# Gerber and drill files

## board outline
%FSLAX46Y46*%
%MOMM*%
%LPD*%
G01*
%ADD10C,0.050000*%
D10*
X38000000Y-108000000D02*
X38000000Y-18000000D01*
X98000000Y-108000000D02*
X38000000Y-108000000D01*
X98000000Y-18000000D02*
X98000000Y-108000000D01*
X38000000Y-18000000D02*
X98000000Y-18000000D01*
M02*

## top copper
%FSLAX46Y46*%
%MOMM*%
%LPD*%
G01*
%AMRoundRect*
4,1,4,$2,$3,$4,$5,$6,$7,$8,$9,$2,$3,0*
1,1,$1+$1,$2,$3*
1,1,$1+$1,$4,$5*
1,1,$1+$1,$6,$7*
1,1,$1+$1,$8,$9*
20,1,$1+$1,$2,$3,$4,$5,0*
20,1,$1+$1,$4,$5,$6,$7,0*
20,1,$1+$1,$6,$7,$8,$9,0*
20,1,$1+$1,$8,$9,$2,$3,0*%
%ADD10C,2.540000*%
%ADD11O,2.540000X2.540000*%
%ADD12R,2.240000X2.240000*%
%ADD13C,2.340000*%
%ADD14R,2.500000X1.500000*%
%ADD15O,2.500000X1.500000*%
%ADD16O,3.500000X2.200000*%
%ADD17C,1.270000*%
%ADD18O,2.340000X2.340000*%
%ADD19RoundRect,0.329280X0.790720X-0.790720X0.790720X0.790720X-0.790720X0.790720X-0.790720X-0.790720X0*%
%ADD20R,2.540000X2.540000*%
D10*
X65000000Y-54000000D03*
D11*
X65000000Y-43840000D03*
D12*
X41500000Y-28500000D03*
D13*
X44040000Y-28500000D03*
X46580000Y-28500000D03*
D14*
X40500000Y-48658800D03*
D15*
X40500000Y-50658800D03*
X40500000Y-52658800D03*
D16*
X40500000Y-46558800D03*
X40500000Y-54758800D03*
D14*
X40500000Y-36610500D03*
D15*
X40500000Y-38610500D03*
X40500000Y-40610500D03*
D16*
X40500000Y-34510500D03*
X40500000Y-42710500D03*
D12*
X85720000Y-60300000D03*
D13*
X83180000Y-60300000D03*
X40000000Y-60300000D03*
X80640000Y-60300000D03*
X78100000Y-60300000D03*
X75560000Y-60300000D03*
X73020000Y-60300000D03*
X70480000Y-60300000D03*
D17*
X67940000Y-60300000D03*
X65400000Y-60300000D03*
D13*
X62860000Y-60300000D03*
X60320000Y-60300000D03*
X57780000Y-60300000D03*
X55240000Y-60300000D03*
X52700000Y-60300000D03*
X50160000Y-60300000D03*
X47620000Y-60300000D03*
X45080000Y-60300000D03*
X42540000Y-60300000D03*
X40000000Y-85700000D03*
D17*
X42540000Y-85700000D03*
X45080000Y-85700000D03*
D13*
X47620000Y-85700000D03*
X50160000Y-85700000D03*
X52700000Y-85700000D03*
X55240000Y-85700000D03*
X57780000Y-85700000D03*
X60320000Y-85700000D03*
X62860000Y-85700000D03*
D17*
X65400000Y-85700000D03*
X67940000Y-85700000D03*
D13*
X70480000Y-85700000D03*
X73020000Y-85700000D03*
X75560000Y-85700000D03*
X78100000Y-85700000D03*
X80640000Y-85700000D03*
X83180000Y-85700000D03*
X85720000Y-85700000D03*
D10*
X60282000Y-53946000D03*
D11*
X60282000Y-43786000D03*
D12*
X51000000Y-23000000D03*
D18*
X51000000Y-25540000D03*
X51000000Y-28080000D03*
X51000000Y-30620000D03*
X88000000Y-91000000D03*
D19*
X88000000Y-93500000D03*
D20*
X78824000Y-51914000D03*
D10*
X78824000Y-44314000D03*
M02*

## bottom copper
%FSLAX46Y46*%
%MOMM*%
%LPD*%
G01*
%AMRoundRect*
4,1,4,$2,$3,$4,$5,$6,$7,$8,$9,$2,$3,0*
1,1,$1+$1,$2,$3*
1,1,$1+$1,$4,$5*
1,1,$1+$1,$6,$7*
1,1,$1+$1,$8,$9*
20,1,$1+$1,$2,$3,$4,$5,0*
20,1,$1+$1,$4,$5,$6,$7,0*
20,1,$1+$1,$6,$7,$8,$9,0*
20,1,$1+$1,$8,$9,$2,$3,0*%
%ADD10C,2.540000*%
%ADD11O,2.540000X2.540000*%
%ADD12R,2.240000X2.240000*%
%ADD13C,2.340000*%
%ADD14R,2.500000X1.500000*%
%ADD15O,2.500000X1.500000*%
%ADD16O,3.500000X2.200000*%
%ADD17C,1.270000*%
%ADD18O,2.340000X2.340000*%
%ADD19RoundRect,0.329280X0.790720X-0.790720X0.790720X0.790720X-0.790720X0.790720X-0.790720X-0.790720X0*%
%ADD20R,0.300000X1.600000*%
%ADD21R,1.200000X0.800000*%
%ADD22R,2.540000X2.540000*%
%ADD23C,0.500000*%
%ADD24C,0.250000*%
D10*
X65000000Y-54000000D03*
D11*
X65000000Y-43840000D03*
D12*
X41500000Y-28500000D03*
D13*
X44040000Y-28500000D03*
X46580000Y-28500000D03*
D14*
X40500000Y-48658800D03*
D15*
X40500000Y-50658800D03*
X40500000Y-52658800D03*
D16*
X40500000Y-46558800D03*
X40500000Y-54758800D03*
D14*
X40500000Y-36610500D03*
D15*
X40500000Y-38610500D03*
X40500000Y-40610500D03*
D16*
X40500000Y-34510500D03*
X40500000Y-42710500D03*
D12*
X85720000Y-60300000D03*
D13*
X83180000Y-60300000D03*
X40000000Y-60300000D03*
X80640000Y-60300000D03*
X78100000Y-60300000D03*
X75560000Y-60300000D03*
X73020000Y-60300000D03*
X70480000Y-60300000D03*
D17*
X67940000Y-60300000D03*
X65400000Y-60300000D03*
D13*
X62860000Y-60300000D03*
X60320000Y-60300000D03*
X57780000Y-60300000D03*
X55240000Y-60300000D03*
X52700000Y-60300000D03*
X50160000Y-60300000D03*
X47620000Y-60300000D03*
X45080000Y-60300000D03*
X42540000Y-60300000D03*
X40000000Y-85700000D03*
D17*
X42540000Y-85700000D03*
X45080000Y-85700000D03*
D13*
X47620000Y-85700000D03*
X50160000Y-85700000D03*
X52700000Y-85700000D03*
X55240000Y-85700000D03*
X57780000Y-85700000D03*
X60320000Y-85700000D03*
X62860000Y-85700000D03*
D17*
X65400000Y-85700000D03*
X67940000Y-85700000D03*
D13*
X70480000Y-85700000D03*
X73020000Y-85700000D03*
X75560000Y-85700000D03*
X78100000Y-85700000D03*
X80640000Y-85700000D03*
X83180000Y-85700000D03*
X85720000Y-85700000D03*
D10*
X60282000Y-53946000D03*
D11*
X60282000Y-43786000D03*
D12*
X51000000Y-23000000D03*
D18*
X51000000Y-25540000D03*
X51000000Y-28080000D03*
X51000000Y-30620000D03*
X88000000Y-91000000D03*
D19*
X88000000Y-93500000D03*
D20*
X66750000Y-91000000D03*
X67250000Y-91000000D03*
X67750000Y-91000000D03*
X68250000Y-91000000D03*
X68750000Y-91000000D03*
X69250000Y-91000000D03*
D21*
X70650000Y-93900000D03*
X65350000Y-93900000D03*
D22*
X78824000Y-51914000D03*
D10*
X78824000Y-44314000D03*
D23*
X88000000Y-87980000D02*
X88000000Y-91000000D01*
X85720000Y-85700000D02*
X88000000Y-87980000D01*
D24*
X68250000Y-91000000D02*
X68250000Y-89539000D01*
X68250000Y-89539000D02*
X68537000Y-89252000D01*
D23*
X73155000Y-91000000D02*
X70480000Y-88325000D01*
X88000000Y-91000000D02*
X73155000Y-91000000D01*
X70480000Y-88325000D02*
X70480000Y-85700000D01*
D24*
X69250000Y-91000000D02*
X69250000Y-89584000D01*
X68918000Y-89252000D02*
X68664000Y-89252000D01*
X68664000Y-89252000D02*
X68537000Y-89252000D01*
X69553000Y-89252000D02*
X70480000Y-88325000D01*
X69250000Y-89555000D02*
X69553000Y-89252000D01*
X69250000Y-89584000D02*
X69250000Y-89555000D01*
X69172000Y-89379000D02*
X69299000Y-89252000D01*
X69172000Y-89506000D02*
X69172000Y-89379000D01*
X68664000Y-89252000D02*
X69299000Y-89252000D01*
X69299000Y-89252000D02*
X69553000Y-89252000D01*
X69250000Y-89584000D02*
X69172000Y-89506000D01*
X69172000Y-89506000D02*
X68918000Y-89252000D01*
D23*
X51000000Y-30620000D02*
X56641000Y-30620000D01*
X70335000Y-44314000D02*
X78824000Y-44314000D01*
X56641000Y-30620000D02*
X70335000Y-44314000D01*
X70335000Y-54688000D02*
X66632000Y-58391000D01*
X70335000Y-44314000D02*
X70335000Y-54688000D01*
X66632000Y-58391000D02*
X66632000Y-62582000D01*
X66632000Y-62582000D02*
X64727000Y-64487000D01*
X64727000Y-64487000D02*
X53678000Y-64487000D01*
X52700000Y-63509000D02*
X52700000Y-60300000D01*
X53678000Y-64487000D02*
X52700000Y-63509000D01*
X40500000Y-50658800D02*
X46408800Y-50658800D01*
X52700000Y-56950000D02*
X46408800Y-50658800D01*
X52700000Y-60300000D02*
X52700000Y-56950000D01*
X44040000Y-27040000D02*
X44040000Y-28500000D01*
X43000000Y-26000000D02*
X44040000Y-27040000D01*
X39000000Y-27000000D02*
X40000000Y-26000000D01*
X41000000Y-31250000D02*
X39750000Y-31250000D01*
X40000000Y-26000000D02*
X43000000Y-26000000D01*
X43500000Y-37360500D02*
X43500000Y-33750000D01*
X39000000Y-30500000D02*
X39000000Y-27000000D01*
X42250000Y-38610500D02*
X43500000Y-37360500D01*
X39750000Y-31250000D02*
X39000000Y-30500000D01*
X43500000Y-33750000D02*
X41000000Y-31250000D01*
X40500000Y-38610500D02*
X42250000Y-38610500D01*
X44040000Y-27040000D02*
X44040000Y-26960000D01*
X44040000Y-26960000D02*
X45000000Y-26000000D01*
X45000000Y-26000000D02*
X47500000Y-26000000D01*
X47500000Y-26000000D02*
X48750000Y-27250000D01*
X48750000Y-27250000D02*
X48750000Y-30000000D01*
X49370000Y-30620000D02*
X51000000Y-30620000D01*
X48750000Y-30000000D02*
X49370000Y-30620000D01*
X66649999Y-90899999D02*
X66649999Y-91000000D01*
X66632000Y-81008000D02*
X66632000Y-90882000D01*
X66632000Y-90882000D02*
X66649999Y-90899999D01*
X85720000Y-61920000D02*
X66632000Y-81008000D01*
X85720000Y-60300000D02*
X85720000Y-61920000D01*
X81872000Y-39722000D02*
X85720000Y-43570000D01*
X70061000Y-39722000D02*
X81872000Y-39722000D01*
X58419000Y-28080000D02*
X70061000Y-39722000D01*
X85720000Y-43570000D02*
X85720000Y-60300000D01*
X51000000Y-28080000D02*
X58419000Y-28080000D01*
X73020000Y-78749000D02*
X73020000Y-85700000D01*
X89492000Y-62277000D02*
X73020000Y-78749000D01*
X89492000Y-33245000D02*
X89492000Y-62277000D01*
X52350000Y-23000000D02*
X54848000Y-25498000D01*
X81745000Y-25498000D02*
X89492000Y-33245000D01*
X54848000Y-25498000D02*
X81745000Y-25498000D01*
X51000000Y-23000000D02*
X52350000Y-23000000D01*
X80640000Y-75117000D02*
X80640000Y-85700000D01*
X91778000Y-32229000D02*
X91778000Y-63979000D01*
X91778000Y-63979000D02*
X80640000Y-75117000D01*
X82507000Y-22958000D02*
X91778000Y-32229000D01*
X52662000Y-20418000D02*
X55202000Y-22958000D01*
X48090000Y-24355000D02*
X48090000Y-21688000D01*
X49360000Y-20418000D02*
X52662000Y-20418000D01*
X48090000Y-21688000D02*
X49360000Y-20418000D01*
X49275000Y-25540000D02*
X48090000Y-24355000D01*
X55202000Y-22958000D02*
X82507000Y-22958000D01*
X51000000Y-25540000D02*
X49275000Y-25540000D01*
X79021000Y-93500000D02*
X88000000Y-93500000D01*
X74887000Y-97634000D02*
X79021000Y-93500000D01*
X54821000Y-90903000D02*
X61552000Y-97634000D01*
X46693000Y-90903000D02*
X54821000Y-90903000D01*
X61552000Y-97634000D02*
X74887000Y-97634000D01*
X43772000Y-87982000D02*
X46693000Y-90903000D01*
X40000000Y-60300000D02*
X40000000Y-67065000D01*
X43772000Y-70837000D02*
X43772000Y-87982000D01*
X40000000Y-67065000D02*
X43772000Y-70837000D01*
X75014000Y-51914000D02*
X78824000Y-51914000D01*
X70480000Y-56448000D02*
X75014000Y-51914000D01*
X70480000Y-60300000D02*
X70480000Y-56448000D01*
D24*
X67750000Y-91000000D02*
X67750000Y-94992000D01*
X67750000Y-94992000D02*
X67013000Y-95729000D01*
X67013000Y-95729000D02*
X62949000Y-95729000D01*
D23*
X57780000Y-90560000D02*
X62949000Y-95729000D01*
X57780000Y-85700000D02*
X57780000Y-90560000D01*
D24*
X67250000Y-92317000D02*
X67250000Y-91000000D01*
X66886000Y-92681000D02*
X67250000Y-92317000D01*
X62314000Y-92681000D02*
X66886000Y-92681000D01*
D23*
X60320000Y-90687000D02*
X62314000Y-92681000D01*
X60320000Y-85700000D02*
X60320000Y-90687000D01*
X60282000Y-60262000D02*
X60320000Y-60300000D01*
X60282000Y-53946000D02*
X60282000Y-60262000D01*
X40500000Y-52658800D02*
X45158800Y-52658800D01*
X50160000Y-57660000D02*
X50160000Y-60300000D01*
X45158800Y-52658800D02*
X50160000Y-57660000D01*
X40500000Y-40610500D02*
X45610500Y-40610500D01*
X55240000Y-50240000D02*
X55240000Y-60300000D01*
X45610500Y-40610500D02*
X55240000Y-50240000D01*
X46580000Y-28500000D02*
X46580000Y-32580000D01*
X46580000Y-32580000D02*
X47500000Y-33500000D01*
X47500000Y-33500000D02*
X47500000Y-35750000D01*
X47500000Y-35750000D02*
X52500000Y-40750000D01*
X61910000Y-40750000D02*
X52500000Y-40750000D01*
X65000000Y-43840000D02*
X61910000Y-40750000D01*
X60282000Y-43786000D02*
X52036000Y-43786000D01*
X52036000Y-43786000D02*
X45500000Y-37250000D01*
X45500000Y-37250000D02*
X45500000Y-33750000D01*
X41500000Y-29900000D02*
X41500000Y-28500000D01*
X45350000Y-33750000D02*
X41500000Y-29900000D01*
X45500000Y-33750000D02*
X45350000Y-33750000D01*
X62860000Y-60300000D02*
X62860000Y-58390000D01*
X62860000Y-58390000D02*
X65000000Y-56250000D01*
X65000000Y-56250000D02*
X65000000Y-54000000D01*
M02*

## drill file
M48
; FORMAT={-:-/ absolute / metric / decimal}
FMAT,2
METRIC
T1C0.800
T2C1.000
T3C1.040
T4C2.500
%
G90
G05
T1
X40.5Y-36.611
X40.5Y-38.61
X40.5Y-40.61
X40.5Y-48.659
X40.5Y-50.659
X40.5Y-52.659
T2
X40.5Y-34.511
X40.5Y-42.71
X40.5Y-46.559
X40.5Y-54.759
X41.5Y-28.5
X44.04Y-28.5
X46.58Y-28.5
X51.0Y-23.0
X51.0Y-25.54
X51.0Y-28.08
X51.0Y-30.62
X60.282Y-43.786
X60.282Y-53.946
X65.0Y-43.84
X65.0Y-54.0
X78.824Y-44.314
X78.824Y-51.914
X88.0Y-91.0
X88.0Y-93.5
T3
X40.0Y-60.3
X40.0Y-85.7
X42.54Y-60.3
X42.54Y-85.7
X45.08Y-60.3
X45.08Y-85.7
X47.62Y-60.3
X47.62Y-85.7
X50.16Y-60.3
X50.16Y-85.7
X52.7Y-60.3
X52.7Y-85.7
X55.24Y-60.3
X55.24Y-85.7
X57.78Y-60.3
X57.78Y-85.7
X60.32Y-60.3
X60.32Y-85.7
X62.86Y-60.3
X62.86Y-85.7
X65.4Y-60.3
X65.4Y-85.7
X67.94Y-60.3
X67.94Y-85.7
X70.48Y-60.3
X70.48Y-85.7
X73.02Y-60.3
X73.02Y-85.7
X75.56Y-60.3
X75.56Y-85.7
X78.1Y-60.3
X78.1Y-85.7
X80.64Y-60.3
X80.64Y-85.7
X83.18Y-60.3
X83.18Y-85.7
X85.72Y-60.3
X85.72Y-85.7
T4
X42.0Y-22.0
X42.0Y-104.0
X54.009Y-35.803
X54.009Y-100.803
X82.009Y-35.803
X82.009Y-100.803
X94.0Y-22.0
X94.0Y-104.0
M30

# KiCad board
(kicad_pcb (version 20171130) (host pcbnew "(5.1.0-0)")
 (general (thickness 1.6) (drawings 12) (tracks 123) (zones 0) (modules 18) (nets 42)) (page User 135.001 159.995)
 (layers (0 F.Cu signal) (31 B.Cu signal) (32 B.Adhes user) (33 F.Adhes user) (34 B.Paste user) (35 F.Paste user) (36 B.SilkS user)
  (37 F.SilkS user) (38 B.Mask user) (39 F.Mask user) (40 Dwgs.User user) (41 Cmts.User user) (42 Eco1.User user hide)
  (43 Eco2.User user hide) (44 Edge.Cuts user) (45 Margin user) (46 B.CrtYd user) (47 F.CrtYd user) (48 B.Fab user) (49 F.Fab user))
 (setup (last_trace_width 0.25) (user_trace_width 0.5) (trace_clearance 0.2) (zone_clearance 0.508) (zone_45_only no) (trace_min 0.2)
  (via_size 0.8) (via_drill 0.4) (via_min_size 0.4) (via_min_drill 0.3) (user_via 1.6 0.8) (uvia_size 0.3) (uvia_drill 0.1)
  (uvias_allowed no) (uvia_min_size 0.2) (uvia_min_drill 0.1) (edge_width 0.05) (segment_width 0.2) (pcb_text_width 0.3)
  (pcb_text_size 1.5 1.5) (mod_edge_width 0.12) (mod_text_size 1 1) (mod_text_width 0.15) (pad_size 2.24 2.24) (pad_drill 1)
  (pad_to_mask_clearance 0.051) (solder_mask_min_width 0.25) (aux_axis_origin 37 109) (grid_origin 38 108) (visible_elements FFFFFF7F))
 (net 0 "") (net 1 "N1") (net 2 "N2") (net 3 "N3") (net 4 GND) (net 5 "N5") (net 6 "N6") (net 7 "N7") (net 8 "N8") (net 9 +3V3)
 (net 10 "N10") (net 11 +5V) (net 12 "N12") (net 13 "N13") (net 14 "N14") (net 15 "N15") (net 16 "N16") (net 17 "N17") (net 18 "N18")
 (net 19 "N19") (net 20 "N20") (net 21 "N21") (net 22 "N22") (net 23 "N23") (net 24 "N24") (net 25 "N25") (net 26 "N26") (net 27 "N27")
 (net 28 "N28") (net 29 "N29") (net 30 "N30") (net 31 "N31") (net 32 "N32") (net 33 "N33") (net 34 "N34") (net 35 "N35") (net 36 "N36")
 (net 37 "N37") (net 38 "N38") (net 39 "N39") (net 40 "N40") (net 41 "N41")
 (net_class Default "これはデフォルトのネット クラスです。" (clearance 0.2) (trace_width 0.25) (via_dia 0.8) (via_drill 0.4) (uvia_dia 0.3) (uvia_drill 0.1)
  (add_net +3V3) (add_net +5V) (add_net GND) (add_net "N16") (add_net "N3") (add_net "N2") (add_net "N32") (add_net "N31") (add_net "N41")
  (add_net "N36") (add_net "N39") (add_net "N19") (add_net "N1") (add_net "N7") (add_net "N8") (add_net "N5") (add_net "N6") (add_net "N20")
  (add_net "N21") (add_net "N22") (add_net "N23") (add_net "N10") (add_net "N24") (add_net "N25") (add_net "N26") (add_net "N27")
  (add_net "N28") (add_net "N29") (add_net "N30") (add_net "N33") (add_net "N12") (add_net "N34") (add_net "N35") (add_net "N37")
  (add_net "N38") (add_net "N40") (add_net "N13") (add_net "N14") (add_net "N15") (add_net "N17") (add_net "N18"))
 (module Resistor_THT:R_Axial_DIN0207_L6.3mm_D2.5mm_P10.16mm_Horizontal (layer F.Cu) (at 65 54 90)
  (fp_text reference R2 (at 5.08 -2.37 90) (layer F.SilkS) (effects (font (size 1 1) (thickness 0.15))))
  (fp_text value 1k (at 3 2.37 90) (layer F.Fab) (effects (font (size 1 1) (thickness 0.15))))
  (pad 1 thru_hole circle (at 0 0 90) (size 2.54 2.54) (drill 1) (layers *.Cu *.Mask) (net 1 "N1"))
  (pad 2 thru_hole oval (at 10.16 0 90) (size 2.54 2.54) (drill 1) (layers *.Cu *.Mask) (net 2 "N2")))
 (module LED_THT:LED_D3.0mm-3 (layer F.Cu) (at 41.5 28.5)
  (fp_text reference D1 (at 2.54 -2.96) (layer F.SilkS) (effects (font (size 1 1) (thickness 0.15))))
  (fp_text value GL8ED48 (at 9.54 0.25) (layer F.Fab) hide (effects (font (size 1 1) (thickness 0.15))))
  (pad 1 thru_hole rect (at 0 0) (size 2.24 2.24) (drill 1) (layers *.Cu *.Mask) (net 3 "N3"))
  (pad 2 thru_hole circle (at 2.54 0) (size 2.34 2.34) (drill 1) (layers *.Cu *.Mask) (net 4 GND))
  (pad 3 thru_hole circle (at 5.08 0) (size 2.34 2.34) (drill 1) (layers *.Cu *.Mask) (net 2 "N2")))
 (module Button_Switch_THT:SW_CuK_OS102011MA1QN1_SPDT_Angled (layer F.Cu) (at 40.5 48.6588 270)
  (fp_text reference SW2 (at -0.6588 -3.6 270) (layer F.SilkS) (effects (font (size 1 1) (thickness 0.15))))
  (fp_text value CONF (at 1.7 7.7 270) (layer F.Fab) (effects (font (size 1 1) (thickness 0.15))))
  (pad 1 thru_hole rect (at 0 0 270) (size 1.5 2.5) (drill 0.8) (layers *.Cu *.Mask) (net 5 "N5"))
  (pad 2 thru_hole oval (at 2 0 270) (size 1.5 2.5) (drill 0.8) (layers *.Cu *.Mask) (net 4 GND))
  (pad 3 thru_hole oval (at 4 0 270) (size 1.5 2.5) (drill 0.8) (layers *.Cu *.Mask) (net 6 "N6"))
  (pad "" thru_hole oval (at -2.1 0 270) (size 2.2 3.5) (drill 1) (layers *.Cu *.Mask))
  (pad "" thru_hole oval (at 6.1 0 270) (size 2.2 3.5) (drill 1) (layers *.Cu *.Mask)))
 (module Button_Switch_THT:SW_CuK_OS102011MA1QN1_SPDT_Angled (layer F.Cu) (at 40.5 36.6105 270)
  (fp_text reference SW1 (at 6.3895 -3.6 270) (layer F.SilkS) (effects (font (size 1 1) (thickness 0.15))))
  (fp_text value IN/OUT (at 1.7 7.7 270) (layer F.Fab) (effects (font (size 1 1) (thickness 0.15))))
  (pad 1 thru_hole rect (at 0 0 270) (size 1.5 2.5) (drill 0.8) (layers *.Cu *.Mask) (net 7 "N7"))
  (pad 2 thru_hole oval (at 2 0 270) (size 1.5 2.5) (drill 0.8) (layers *.Cu *.Mask) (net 4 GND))
  (pad 3 thru_hole oval (at 4 0 270) (size 1.5 2.5) (drill 0.8) (layers *.Cu *.Mask) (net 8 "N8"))
  (pad "" thru_hole oval (at -2.1 0 270) (size 2.2 3.5) (drill 1) (layers *.Cu *.Mask))
  (pad "" thru_hole oval (at 6.1 0 270) (size 2.2 3.5) (drill 1) (layers *.Cu *.Mask)))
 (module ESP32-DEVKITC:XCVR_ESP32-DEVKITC (layer F.Cu) (at 66.26 73 270)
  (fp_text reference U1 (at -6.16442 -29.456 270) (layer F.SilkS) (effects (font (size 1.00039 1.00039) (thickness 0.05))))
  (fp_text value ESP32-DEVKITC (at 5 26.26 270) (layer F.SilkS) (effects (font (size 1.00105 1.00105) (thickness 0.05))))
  (pad 1 thru_hole rect (at -12.7 -19.46 270) (size 2.24 2.24) (drill 1.04) (layers *.Cu *.Mask) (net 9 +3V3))
  (pad 2 thru_hole circle (at -12.7 -16.92 270) (size 2.34 2.34) (drill 1.04) (layers *.Cu *.Mask) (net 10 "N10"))
  (pad 19 thru_hole circle (at -12.7 26.26 270) (size 2.34 2.34) (drill 1.04) (layers *.Cu *.Mask) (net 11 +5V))
  (pad 3 thru_hole circle (at -12.7 -14.38 270) (size 2.34 2.34) (drill 1.04) (layers *.Cu *.Mask) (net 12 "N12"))
  (pad 4 thru_hole circle (at -12.7 -11.84 270) (size 2.34 2.34) (drill 1.04) (layers *.Cu *.Mask) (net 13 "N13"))
  (pad 5 thru_hole circle (at -12.7 -9.3 270) (size 2.34 2.34) (drill 1.04) (layers *.Cu *.Mask) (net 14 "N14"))
  (pad 6 thru_hole circle (at -12.7 -6.76 270) (size 2.34 2.34) (drill 1.04) (layers *.Cu *.Mask) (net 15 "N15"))
  (pad 7 thru_hole circle (at -12.7 -4.22 270) (size 2.34 2.34) (drill 1.04) (layers *.Cu *.Mask) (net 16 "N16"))
  (pad 8 thru_hole circle (at -12.7 -1.68 270) (size 1.27 1.27) (drill 1.04) (layers *.Cu *.Mask) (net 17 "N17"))
  (pad 9 thru_hole circle (at -12.7 0.86 270) (size 1.27 1.27) (drill 1.04) (layers *.Cu *.Mask) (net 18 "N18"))
  (pad 10 thru_hole circle (at -12.7 3.4 270) (size 2.34 2.34) (drill 1.04) (layers *.Cu *.Mask) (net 1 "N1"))
  (pad 11 thru_hole circle (at -12.7 5.94 270) (size 2.34 2.34) (drill 1.04) (layers *.Cu *.Mask) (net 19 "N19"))
  (pad 12 thru_hole circle (at -12.7 8.48 270) (size 2.34 2.34) (drill 1.04) (layers *.Cu *.Mask) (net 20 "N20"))
  (pad 13 thru_hole circle (at -12.7 11.02 270) (size 2.34 2.34) (drill 1.04) (layers *.Cu *.Mask) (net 8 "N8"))
  (pad 14 thru_hole circle (at -12.7 13.56 270) (size 2.34 2.34) (drill 1.04) (layers *.Cu *.Mask) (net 4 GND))
  (pad 15 thru_hole circle (at -12.7 16.1 270) (size 2.34 2.34) (drill 1.04) (layers *.Cu *.Mask) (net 6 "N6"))
  (pad 16 thru_hole circle (at -12.7 18.64 270) (size 2.34 2.34) (drill 1.04) (layers *.Cu *.Mask) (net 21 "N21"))
  (pad 17 thru_hole circle (at -12.7 21.18 270) (size 2.34 2.34) (drill 1.04) (layers *.Cu *.Mask) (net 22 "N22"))
  (pad 18 thru_hole circle (at -12.7 23.72 270) (size 2.34 2.34) (drill 1.04) (layers *.Cu *.Mask) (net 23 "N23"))
  (pad 20 thru_hole circle (at 12.7 26.26 90) (size 2.34 2.34) (drill 1.04) (layers *.Cu *.Mask) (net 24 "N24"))
  (pad 21 thru_hole circle (at 12.7 23.72 90) (size 1.27 1.27) (drill 1.04) (layers *.Cu *.Mask) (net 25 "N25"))
  (pad 22 thru_hole circle (at 12.7 21.18 90) (size 1.27 1.27) (drill 1.04) (layers *.Cu *.Mask) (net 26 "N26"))
  (pad 23 thru_hole circle (at 12.7 18.64 90) (size 2.34 2.34) (drill 1.04) (layers *.Cu *.Mask) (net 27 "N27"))
  (pad 24 thru_hole circle (at 12.7 16.1 90) (size 2.34 2.34) (drill 1.04) (layers *.Cu *.Mask) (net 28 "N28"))
  (pad 25 thru_hole circle (at 12.7 13.56 90) (size 2.34 2.34) (drill 1.04) (layers *.Cu *.Mask) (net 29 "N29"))
  (pad 26 thru_hole circle (at 12.7 11.02 90) (size 2.34 2.34) (drill 1.04) (layers *.Cu *.Mask) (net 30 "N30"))
  (pad 27 thru_hole circle (at 12.7 8.48 90) (size 2.34 2.34) (drill 1.04) (layers *.Cu *.Mask) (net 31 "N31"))
  (pad 28 thru_hole circle (at 12.7 5.94 90) (size 2.34 2.34) (drill 1.04) (layers *.Cu *.Mask) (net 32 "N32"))
  (pad 29 thru_hole circle (at 12.7 3.4 90) (size 2.34 2.34) (drill 1.04) (layers *.Cu *.Mask) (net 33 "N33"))
  (pad 30 thru_hole circle (at 12.7 0.86 90) (size 1.27 1.27) (drill 1.04) (layers *.Cu *.Mask) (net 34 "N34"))
  (pad 31 thru_hole circle (at 12.7 -1.68 90) (size 1.27 1.27) (drill 1.04) (layers *.Cu *.Mask) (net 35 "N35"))
  (pad 32 thru_hole circle (at 12.7 -4.22 90) (size 2.34 2.34) (drill 1.04) (layers *.Cu *.Mask) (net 4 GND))
  (pad 33 thru_hole circle (at 12.7 -6.76 90) (size 2.34 2.34) (drill 1.04) (layers *.Cu *.Mask) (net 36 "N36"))
  (pad 34 thru_hole circle (at 12.7 -9.3 90) (size 2.34 2.34) (drill 1.04) (layers *.Cu *.Mask) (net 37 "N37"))
  (pad 35 thru_hole circle (at 12.7 -11.84 90) (size 2.34 2.34) (drill 1.04) (layers *.Cu *.Mask) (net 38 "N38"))
  (pad 36 thru_hole circle (at 12.7 -14.38 90) (size 2.34 2.34) (drill 1.04) (layers *.Cu *.Mask) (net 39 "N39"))
  (pad 37 thru_hole circle (at 12.7 -16.92 90) (size 2.34 2.34) (drill 1.04) (layers *.Cu *.Mask) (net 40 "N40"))
  (pad 38 thru_hole circle (at 12.7 -19.46 90) (size 2.34 2.34) (drill 1.04) (layers *.Cu *.Mask) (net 4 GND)))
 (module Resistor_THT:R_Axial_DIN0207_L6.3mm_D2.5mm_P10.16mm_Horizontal (layer F.Cu) (at 60.282 53.946 90)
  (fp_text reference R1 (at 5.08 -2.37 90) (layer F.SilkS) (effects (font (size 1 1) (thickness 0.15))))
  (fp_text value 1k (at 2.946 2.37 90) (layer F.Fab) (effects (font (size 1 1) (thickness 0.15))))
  (pad 1 thru_hole circle (at 0 0 90) (size 2.54 2.54) (drill 1) (layers *.Cu *.Mask) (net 19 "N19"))
  (pad 2 thru_hole oval (at 10.16 0 90) (size 2.54 2.54) (drill 1) (layers *.Cu *.Mask) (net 3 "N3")))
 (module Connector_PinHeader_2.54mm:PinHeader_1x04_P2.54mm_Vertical (layer F.Cu) (at 51 23)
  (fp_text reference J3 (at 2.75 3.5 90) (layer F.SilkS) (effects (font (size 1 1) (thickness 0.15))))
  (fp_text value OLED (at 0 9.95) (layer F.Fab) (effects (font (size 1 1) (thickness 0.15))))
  (pad 1 thru_hole rect (at 0 0) (size 2.24 2.24) (drill 1) (layers *.Cu *.Mask) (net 36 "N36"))
  (pad 2 thru_hole oval (at 0 2.54) (size 2.34 2.34) (drill 1) (layers *.Cu *.Mask) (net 39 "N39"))
  (pad 3 thru_hole oval (at 0 5.08) (size 2.34 2.34) (drill 1) (layers *.Cu *.Mask) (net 9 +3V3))
  (pad 4 thru_hole oval (at 0 7.62) (size 2.34 2.34) (drill 1) (layers *.Cu *.Mask) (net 4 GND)))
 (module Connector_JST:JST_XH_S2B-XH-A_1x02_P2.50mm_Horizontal (layer F.Cu) (at 88 93.5 90)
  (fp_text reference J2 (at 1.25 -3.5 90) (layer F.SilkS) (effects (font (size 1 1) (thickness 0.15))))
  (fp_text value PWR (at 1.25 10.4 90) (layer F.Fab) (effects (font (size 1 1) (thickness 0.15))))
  (pad 2 thru_hole oval (at 2.5 0 90) (size 2.34 2.34) (drill 1) (layers *.Cu *.Mask) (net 4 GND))
  (pad 1 thru_hole roundrect (at 0 0 90) (size 2.24 2.24) (drill 1) (layers *.Cu *.Mask) (roundrect_rratio 0.147) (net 11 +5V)))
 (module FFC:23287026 (layer B.Cu) (at 68 92.8 180)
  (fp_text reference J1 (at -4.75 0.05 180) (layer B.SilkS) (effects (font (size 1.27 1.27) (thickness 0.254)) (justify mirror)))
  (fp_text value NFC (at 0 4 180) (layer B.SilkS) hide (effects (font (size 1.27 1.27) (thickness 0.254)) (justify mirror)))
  (pad 1 smd rect (at 1.25 1.8 180) (size 0.3 1.6) (layers B.Cu B.Paste B.Mask) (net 9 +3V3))
  (pad 2 smd rect (at 0.75 1.8 180) (size 0.3 1.6) (layers B.Cu B.Paste B.Mask) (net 32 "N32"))
  (pad 3 smd rect (at 0.25 1.8 180) (size 0.3 1.6) (layers B.Cu B.Paste B.Mask) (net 31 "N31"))
  (pad 4 smd rect (at -0.25 1.8 180) (size 0.3 1.6) (layers B.Cu B.Paste B.Mask) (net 4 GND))
  (pad 5 smd rect (at -0.75 1.8 180) (size 0.3 1.6) (layers B.Cu B.Paste B.Mask) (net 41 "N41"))
  (pad 6 smd rect (at -1.25 1.8 180) (size 0.3 1.6) (layers B.Cu B.Paste B.Mask) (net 4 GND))
  (pad MP1 smd rect (at -2.65 -1.1 180) (size 1.2 0.8) (layers B.Cu B.Paste B.Mask))
  (pad MP2 smd rect (at 2.65 -1.1 180) (size 1.2 0.8) (layers B.Cu B.Paste B.Mask)))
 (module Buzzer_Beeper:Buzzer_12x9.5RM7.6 (layer F.Cu) (at 78.824 51.914 90)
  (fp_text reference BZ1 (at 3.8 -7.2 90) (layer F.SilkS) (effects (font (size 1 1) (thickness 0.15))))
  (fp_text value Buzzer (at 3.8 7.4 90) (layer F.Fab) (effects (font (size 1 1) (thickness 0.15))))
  (pad 1 thru_hole rect (at 0 0 90) (size 2.54 2.54) (drill 1) (layers *.Cu *.Mask) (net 16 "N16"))
  (pad 2 thru_hole circle (at 7.6 0 90) (size 2.54 2.54) (drill 1) (layers *.Cu *.Mask) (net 4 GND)))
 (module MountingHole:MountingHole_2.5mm (layer F.Cu) (at 42 104)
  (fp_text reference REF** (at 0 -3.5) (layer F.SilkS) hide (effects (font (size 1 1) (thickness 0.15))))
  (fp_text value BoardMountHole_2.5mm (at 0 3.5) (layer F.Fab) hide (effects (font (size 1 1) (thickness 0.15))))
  (pad 1 np_thru_hole circle (at 0 0) (size 2.5 2.5) (drill 2.5) (layers *.Cu *.Mask)))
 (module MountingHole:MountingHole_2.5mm (layer F.Cu) (at 94 104)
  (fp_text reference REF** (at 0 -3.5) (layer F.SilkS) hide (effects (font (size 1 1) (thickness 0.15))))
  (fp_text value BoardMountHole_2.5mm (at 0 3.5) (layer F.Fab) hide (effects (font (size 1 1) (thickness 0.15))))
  (pad 1 np_thru_hole circle (at 0 0) (size 2.5 2.5) (drill 2.5) (layers *.Cu *.Mask)))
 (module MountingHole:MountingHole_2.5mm (layer F.Cu) (at 94 22)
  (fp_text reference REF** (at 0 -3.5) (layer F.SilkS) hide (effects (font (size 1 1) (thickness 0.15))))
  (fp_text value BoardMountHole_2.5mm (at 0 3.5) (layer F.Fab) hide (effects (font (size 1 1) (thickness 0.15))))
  (pad 1 np_thru_hole circle (at 0 0) (size 2.5 2.5) (drill 2.5) (layers *.Cu *.Mask)))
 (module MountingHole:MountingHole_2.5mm (layer F.Cu) (at 42 22)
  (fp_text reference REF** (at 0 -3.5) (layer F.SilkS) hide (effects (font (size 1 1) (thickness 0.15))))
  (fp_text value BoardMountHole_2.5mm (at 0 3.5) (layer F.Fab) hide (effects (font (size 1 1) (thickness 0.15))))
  (pad 1 np_thru_hole circle (at 0 0) (size 2.5 2.5) (drill 2.5) (layers *.Cu *.Mask)))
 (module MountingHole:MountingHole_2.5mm (layer F.Cu) (at 54.008576 35.802609 90)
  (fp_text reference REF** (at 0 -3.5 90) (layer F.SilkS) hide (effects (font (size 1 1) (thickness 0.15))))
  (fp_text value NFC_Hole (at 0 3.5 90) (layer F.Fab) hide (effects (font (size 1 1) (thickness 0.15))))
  (pad 1 np_thru_hole circle (at 0 0 90) (size 2.5 2.5) (drill 2.5) (layers *.Cu *.Mask)))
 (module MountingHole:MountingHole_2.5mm (layer F.Cu) (at 82.008576 100.802609 90)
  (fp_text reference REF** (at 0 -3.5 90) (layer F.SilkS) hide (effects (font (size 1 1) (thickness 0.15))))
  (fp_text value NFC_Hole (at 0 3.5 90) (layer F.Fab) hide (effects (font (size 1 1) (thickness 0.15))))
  (pad 1 np_thru_hole circle (at 0 0 90) (size 2.5 2.5) (drill 2.5) (layers *.Cu *.Mask)))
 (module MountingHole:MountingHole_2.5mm (layer F.Cu) (at 82.008576 35.802609 90)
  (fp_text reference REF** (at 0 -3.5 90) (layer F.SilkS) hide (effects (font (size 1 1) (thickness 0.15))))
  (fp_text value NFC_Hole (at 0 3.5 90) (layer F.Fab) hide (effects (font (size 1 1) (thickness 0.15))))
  (pad 1 np_thru_hole circle (at 0 0 90) (size 2.5 2.5) (drill 2.5) (layers *.Cu *.Mask)))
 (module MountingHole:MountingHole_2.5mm (layer F.Cu) (at 54.008576 100.802609 90)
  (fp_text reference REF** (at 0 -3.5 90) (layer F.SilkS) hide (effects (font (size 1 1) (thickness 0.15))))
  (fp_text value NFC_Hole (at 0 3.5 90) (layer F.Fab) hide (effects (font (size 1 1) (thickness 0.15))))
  (pad 1 np_thru_hole circle (at 0 0 90) (size 2.5 2.5) (drill 2.5) (layers *.Cu *.Mask)))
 (gr_line (start 38 108) (end 38 18) (layer Edge.Cuts) (width 0.05))
 (gr_line (start 98 108) (end 38 108) (layer Edge.Cuts) (width 0.05))
 (gr_line (start 98 18) (end 98 108) (layer Edge.Cuts) (width 0.05))
 (gr_line (start 38 18) (end 98 18) (layer Edge.Cuts) (width 0.05))
 (segment (start 88 87.98) (end 88 91) (width 0.5) (layer B.Cu) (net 4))
 (segment (start 85.72 85.7) (end 88 87.98) (width 0.5) (layer B.Cu) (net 4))
 (segment (start 68.25 91) (end 68.25 89.539) (width 0.25) (layer B.Cu) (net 4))
 (segment (start 68.25 89.539) (end 68.537 89.252) (width 0.25) (layer B.Cu) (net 4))
 (segment (start 73.155 91) (end 70.48 88.325) (width 0.5) (layer B.Cu) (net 4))
 (segment (start 88 91) (end 73.155 91) (width 0.5) (layer B.Cu) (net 4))
 (segment (start 70.48 88.325) (end 70.48 85.7) (width 0.5) (layer B.Cu) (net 4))
 (segment (start 69.25 91) (end 69.25 89.584) (width 0.25) (layer B.Cu) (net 4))
 (segment (start 68.918 89.252) (end 68.664 89.252) (width 0.25) (layer B.Cu) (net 4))
 (segment (start 68.664 89.252) (end 68.537 89.252) (width 0.25) (layer B.Cu) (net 4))
 (segment (start 69.553 89.252) (end 70.48 88.325) (width 0.25) (layer B.Cu) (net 4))
 (segment (start 69.25 89.555) (end 69.553 89.252) (width 0.25) (layer B.Cu) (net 4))
 (segment (start 69.25 89.584) (end 69.25 89.555) (width 0.25) (layer B.Cu) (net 4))
 (segment (start 69.172 89.379) (end 69.299 89.252) (width 0.25) (layer B.Cu) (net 4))
 (segment (start 69.172 89.506) (end 69.172 89.379) (width 0.25) (layer B.Cu) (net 4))
 (segment (start 68.664 89.252) (end 69.299 89.252) (width 0.25) (layer B.Cu) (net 4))
 (segment (start 69.299 89.252) (end 69.553 89.252) (width 0.25) (layer B.Cu) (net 4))
 (segment (start 69.25 89.584) (end 69.172 89.506) (width 0.25) (layer B.Cu) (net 4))
 (segment (start 69.172 89.506) (end 68.918 89.252) (width 0.25) (layer B.Cu) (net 4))
 (segment (start 51 30.62) (end 56.641 30.62) (width 0.5) (layer B.Cu) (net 4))
 (segment (start 70.335 44.314) (end 78.824 44.314) (width 0.5) (layer B.Cu) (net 4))
 (segment (start 56.641 30.62) (end 70.335 44.314) (width 0.5) (layer B.Cu) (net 4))
 (segment (start 70.335 54.688) (end 66.632 58.391) (width 0.5) (layer B.Cu) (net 4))
 (segment (start 70.335 44.314) (end 70.335 54.688) (width 0.5) (layer B.Cu) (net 4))
 (segment (start 66.632 58.391) (end 66.632 62.582) (width 0.5) (layer B.Cu) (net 4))
 (segment (start 66.632 62.582) (end 64.727 64.487) (width 0.5) (layer B.Cu) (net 4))
 (segment (start 64.727 64.487) (end 53.678 64.487) (width 0.5) (layer B.Cu) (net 4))
 (segment (start 52.7 63.509) (end 52.7 60.3) (width 0.5) (layer B.Cu) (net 4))
 (segment (start 53.678 64.487) (end 52.7 63.509) (width 0.5) (layer B.Cu) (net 4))
 (segment (start 40.5 50.6588) (end 46.4088 50.6588) (width 0.5) (layer B.Cu) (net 4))
 (segment (start 52.7 56.95) (end 46.4088 50.6588) (width 0.5) (layer B.Cu) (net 4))
 (segment (start 52.7 60.3) (end 52.7 56.95) (width 0.5) (layer B.Cu) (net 4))
 (segment (start 44.04 27.04) (end 44.04 28.5) (width 0.5) (layer B.Cu) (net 4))
 (segment (start 43 26) (end 44.04 27.04) (width 0.5) (layer B.Cu) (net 4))
 (segment (start 39 27) (end 40 26) (width 0.5) (layer B.Cu) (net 4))
 (segment (start 41 31.25) (end 39.75 31.25) (width 0.5) (layer B.Cu) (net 4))
 (segment (start 40 26) (end 43 26) (width 0.5) (layer B.Cu) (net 4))
 (segment (start 43.5 37.3605) (end 43.5 33.75) (width 0.5) (layer B.Cu) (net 4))
 (segment (start 39 30.5) (end 39 27) (width 0.5) (layer B.Cu) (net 4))
 (segment (start 42.25 38.6105) (end 43.5 37.3605) (width 0.5) (layer B.Cu) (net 4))
 (segment (start 39.75 31.25) (end 39 30.5) (width 0.5) (layer B.Cu) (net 4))
 (segment (start 43.5 33.75) (end 41 31.25) (width 0.5) (layer B.Cu) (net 4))
 (segment (start 40.5 38.6105) (end 42.25 38.6105) (width 0.5) (layer B.Cu) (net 4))
 (segment (start 44.04 27.04) (end 44.04 26.96) (width 0.5) (layer B.Cu) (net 4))
 (segment (start 44.04 26.96) (end 45 26) (width 0.5) (layer B.Cu) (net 4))
 (segment (start 45 26) (end 47.5 26) (width 0.5) (layer B.Cu) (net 4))
 (segment (start 47.5 26) (end 48.75 27.25) (width 0.5) (layer B.Cu) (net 4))
 (segment (start 48.75 27.25) (end 48.75 30) (width 0.5) (layer B.Cu) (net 4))
 (segment (start 49.37 30.62) (end 51 30.62) (width 0.5) (layer B.Cu) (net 4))
 (segment (start 48.75 30) (end 49.37 30.62) (width 0.5) (layer B.Cu) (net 4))
 (segment (start 66.649999 90.899999) (end 66.649999 91) (width 0.5) (layer B.Cu) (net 9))
 (segment (start 66.632 81.008) (end 66.632 90.882) (width 0.5) (layer B.Cu) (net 9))
 (segment (start 66.632 90.882) (end 66.649999 90.899999) (width 0.5) (layer B.Cu) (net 9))
 (segment (start 85.72 61.92) (end 66.632 81.008) (width 0.5) (layer B.Cu) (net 9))
 (segment (start 85.72 60.3) (end 85.72 61.92) (width 0.5) (layer B.Cu) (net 9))
 (segment (start 81.872 39.722) (end 85.72 43.57) (width 0.5) (layer B.Cu) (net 9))
 (segment (start 70.061 39.722) (end 81.872 39.722) (width 0.5) (layer B.Cu) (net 9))
 (segment (start 58.419 28.08) (end 70.061 39.722) (width 0.5) (layer B.Cu) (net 9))
 (segment (start 85.72 43.57) (end 85.72 60.3) (width 0.5) (layer B.Cu) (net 9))
 (segment (start 51 28.08) (end 58.419 28.08) (width 0.5) (layer B.Cu) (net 9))
 (segment (start 73.02 78.749) (end 73.02 85.7) (width 0.5) (layer B.Cu) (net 36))
 (segment (start 89.492 62.277) (end 73.02 78.749) (width 0.5) (layer B.Cu) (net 36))
 (segment (start 89.492 33.245) (end 89.492 62.277) (width 0.5) (layer B.Cu) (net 36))
 (segment (start 52.35 23) (end 54.848 25.498) (width 0.5) (layer B.Cu) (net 36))
 (segment (start 81.745 25.498) (end 89.492 33.245) (width 0.5) (layer B.Cu) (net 36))
 (segment (start 54.848 25.498) (end 81.745 25.498) (width 0.5) (layer B.Cu) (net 36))
 (segment (start 51 23) (end 52.35 23) (width 0.5) (layer B.Cu) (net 36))
 (segment (start 80.64 75.117) (end 80.64 85.7) (width 0.5) (layer B.Cu) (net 39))
 (segment (start 91.778 32.229) (end 91.778 63.979) (width 0.5) (layer B.Cu) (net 39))
 (segment (start 91.778 63.979) (end 80.64 75.117) (width 0.5) (layer B.Cu) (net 39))
 (segment (start 82.507 22.958) (end 91.778 32.229) (width 0.5) (layer B.Cu) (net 39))
 (segment (start 52.662 20.418) (end 55.202 22.958) (width 0.5) (layer B.Cu) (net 39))
 (segment (start 48.09 24.355) (end 48.09 21.688) (width 0.5) (layer B.Cu) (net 39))
 (segment (start 49.36 20.418) (end 52.662 20.418) (width 0.5) (layer B.Cu) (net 39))
 (segment (start 48.09 21.688) (end 49.36 20.418) (width 0.5) (layer B.Cu) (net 39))
 (segment (start 49.275 25.54) (end 48.09 24.355) (width 0.5) (layer B.Cu) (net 39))
 (segment (start 55.202 22.958) (end 82.507 22.958) (width 0.5) (layer B.Cu) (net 39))
 (segment (start 51 25.54) (end 49.275 25.54) (width 0.5) (layer B.Cu) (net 39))
 (segment (start 79.021 93.5) (end 88 93.5) (width 0.5) (layer B.Cu) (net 11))
 (segment (start 74.887 97.634) (end 79.021 93.5) (width 0.5) (layer B.Cu) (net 11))
 (segment (start 54.821 90.903) (end 61.552 97.634) (width 0.5) (layer B.Cu) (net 11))
 (segment (start 46.693 90.903) (end 54.821 90.903) (width 0.5) (layer B.Cu) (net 11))
 (segment (start 61.552 97.634) (end 74.887 97.634) (width 0.5) (layer B.Cu) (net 11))
 (segment (start 43.772 87.982) (end 46.693 90.903) (width 0.5) (layer B.Cu) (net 11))
 (segment (start 40 60.3) (end 40 67.065) (width 0.5) (layer B.Cu) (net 11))
 (segment (start 43.772 70.837) (end 43.772 87.982) (width 0.5) (layer B.Cu) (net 11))
 (segment (start 40 67.065) (end 43.772 70.837) (width 0.5) (layer B.Cu) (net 11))
 (segment (start 75.014 51.914) (end 78.824 51.914) (width 0.5) (layer B.Cu) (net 16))
 (segment (start 70.48 56.448) (end 75.014 51.914) (width 0.5) (layer B.Cu) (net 16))
 (segment (start 70.48 60.3) (end 70.48 56.448) (width 0.5) (layer B.Cu) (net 16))
 (segment (start 67.75 91) (end 67.75 94.992) (width 0.25) (layer B.Cu) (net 31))
 (segment (start 67.75 94.992) (end 67.013 95.729) (width 0.25) (layer B.Cu) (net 31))
 (segment (start 67.013 95.729) (end 62.949 95.729) (width 0.25) (layer B.Cu) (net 31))
 (segment (start 57.78 90.56) (end 62.949 95.729) (width 0.5) (layer B.Cu) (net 31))
 (segment (start 57.78 85.7) (end 57.78 90.56) (width 0.5) (layer B.Cu) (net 31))
 (segment (start 67.25 92.317) (end 67.25 91) (width 0.25) (layer B.Cu) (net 32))
 (segment (start 66.886 92.681) (end 67.25 92.317) (width 0.25) (layer B.Cu) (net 32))
 (segment (start 62.314 92.681) (end 66.886 92.681) (width 0.25) (layer B.Cu) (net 32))
 (segment (start 60.32 90.687) (end 62.314 92.681) (width 0.5) (layer B.Cu) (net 32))
 (segment (start 60.32 85.7) (end 60.32 90.687) (width 0.5) (layer B.Cu) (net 32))
 (segment (start 60.282 60.262) (end 60.32 60.3) (width 0.5) (layer B.Cu) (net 19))
 (segment (start 60.282 53.946) (end 60.282 60.262) (width 0.5) (layer B.Cu) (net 19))
 (segment (start 40.5 52.6588) (end 45.1588 52.6588) (width 0.5) (layer B.Cu) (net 6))
 (segment (start 50.16 57.66) (end 50.16 60.3) (width 0.5) (layer B.Cu) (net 6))
 (segment (start 45.1588 52.6588) (end 50.16 57.66) (width 0.5) (layer B.Cu) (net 6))
 (segment (start 40.5 40.6105) (end 45.6105 40.6105) (width 0.5) (layer B.Cu) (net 8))
 (segment (start 55.24 50.24) (end 55.24 60.3) (width 0.5) (layer B.Cu) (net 8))
 (segment (start 45.6105 40.6105) (end 55.24 50.24) (width 0.5) (layer B.Cu) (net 8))
 (segment (start 46.58 28.5) (end 46.58 32.58) (width 0.5) (layer B.Cu) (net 2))
 (segment (start 46.58 32.58) (end 47.5 33.5) (width 0.5) (layer B.Cu) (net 2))
 (segment (start 47.5 33.5) (end 47.5 35.75) (width 0.5) (layer B.Cu) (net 2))
 (segment (start 47.5 35.75) (end 52.5 40.75) (width 0.5) (layer B.Cu) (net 2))
 (segment (start 61.91 40.75) (end 52.5 40.75) (width 0.5) (layer B.Cu) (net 2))
 (segment (start 65 43.84) (end 61.91 40.75) (width 0.5) (layer B.Cu) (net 2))
 (segment (start 60.282 43.786) (end 52.036 43.786) (width 0.5) (layer B.Cu) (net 3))
 (segment (start 52.036 43.786) (end 45.5 37.25) (width 0.5) (layer B.Cu) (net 3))
 (segment (start 45.5 37.25) (end 45.5 33.75) (width 0.5) (layer B.Cu) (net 3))
 (segment (start 41.5 29.9) (end 41.5 28.5) (width 0.5) (layer B.Cu) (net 3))
 (segment (start 45.35 33.75) (end 41.5 29.9) (width 0.5) (layer B.Cu) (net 3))
 (segment (start 45.5 33.75) (end 45.35 33.75) (width 0.5) (layer B.Cu) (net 3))
 (segment (start 62.86 60.3) (end 62.86 58.39) (width 0.5) (layer B.Cu) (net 1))
 (segment (start 62.86 58.39) (end 65 56.25) (width 0.5) (layer B.Cu) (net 1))
 (segment (start 65 56.25) (end 65 54) (width 0.5) (layer B.Cu) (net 1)))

